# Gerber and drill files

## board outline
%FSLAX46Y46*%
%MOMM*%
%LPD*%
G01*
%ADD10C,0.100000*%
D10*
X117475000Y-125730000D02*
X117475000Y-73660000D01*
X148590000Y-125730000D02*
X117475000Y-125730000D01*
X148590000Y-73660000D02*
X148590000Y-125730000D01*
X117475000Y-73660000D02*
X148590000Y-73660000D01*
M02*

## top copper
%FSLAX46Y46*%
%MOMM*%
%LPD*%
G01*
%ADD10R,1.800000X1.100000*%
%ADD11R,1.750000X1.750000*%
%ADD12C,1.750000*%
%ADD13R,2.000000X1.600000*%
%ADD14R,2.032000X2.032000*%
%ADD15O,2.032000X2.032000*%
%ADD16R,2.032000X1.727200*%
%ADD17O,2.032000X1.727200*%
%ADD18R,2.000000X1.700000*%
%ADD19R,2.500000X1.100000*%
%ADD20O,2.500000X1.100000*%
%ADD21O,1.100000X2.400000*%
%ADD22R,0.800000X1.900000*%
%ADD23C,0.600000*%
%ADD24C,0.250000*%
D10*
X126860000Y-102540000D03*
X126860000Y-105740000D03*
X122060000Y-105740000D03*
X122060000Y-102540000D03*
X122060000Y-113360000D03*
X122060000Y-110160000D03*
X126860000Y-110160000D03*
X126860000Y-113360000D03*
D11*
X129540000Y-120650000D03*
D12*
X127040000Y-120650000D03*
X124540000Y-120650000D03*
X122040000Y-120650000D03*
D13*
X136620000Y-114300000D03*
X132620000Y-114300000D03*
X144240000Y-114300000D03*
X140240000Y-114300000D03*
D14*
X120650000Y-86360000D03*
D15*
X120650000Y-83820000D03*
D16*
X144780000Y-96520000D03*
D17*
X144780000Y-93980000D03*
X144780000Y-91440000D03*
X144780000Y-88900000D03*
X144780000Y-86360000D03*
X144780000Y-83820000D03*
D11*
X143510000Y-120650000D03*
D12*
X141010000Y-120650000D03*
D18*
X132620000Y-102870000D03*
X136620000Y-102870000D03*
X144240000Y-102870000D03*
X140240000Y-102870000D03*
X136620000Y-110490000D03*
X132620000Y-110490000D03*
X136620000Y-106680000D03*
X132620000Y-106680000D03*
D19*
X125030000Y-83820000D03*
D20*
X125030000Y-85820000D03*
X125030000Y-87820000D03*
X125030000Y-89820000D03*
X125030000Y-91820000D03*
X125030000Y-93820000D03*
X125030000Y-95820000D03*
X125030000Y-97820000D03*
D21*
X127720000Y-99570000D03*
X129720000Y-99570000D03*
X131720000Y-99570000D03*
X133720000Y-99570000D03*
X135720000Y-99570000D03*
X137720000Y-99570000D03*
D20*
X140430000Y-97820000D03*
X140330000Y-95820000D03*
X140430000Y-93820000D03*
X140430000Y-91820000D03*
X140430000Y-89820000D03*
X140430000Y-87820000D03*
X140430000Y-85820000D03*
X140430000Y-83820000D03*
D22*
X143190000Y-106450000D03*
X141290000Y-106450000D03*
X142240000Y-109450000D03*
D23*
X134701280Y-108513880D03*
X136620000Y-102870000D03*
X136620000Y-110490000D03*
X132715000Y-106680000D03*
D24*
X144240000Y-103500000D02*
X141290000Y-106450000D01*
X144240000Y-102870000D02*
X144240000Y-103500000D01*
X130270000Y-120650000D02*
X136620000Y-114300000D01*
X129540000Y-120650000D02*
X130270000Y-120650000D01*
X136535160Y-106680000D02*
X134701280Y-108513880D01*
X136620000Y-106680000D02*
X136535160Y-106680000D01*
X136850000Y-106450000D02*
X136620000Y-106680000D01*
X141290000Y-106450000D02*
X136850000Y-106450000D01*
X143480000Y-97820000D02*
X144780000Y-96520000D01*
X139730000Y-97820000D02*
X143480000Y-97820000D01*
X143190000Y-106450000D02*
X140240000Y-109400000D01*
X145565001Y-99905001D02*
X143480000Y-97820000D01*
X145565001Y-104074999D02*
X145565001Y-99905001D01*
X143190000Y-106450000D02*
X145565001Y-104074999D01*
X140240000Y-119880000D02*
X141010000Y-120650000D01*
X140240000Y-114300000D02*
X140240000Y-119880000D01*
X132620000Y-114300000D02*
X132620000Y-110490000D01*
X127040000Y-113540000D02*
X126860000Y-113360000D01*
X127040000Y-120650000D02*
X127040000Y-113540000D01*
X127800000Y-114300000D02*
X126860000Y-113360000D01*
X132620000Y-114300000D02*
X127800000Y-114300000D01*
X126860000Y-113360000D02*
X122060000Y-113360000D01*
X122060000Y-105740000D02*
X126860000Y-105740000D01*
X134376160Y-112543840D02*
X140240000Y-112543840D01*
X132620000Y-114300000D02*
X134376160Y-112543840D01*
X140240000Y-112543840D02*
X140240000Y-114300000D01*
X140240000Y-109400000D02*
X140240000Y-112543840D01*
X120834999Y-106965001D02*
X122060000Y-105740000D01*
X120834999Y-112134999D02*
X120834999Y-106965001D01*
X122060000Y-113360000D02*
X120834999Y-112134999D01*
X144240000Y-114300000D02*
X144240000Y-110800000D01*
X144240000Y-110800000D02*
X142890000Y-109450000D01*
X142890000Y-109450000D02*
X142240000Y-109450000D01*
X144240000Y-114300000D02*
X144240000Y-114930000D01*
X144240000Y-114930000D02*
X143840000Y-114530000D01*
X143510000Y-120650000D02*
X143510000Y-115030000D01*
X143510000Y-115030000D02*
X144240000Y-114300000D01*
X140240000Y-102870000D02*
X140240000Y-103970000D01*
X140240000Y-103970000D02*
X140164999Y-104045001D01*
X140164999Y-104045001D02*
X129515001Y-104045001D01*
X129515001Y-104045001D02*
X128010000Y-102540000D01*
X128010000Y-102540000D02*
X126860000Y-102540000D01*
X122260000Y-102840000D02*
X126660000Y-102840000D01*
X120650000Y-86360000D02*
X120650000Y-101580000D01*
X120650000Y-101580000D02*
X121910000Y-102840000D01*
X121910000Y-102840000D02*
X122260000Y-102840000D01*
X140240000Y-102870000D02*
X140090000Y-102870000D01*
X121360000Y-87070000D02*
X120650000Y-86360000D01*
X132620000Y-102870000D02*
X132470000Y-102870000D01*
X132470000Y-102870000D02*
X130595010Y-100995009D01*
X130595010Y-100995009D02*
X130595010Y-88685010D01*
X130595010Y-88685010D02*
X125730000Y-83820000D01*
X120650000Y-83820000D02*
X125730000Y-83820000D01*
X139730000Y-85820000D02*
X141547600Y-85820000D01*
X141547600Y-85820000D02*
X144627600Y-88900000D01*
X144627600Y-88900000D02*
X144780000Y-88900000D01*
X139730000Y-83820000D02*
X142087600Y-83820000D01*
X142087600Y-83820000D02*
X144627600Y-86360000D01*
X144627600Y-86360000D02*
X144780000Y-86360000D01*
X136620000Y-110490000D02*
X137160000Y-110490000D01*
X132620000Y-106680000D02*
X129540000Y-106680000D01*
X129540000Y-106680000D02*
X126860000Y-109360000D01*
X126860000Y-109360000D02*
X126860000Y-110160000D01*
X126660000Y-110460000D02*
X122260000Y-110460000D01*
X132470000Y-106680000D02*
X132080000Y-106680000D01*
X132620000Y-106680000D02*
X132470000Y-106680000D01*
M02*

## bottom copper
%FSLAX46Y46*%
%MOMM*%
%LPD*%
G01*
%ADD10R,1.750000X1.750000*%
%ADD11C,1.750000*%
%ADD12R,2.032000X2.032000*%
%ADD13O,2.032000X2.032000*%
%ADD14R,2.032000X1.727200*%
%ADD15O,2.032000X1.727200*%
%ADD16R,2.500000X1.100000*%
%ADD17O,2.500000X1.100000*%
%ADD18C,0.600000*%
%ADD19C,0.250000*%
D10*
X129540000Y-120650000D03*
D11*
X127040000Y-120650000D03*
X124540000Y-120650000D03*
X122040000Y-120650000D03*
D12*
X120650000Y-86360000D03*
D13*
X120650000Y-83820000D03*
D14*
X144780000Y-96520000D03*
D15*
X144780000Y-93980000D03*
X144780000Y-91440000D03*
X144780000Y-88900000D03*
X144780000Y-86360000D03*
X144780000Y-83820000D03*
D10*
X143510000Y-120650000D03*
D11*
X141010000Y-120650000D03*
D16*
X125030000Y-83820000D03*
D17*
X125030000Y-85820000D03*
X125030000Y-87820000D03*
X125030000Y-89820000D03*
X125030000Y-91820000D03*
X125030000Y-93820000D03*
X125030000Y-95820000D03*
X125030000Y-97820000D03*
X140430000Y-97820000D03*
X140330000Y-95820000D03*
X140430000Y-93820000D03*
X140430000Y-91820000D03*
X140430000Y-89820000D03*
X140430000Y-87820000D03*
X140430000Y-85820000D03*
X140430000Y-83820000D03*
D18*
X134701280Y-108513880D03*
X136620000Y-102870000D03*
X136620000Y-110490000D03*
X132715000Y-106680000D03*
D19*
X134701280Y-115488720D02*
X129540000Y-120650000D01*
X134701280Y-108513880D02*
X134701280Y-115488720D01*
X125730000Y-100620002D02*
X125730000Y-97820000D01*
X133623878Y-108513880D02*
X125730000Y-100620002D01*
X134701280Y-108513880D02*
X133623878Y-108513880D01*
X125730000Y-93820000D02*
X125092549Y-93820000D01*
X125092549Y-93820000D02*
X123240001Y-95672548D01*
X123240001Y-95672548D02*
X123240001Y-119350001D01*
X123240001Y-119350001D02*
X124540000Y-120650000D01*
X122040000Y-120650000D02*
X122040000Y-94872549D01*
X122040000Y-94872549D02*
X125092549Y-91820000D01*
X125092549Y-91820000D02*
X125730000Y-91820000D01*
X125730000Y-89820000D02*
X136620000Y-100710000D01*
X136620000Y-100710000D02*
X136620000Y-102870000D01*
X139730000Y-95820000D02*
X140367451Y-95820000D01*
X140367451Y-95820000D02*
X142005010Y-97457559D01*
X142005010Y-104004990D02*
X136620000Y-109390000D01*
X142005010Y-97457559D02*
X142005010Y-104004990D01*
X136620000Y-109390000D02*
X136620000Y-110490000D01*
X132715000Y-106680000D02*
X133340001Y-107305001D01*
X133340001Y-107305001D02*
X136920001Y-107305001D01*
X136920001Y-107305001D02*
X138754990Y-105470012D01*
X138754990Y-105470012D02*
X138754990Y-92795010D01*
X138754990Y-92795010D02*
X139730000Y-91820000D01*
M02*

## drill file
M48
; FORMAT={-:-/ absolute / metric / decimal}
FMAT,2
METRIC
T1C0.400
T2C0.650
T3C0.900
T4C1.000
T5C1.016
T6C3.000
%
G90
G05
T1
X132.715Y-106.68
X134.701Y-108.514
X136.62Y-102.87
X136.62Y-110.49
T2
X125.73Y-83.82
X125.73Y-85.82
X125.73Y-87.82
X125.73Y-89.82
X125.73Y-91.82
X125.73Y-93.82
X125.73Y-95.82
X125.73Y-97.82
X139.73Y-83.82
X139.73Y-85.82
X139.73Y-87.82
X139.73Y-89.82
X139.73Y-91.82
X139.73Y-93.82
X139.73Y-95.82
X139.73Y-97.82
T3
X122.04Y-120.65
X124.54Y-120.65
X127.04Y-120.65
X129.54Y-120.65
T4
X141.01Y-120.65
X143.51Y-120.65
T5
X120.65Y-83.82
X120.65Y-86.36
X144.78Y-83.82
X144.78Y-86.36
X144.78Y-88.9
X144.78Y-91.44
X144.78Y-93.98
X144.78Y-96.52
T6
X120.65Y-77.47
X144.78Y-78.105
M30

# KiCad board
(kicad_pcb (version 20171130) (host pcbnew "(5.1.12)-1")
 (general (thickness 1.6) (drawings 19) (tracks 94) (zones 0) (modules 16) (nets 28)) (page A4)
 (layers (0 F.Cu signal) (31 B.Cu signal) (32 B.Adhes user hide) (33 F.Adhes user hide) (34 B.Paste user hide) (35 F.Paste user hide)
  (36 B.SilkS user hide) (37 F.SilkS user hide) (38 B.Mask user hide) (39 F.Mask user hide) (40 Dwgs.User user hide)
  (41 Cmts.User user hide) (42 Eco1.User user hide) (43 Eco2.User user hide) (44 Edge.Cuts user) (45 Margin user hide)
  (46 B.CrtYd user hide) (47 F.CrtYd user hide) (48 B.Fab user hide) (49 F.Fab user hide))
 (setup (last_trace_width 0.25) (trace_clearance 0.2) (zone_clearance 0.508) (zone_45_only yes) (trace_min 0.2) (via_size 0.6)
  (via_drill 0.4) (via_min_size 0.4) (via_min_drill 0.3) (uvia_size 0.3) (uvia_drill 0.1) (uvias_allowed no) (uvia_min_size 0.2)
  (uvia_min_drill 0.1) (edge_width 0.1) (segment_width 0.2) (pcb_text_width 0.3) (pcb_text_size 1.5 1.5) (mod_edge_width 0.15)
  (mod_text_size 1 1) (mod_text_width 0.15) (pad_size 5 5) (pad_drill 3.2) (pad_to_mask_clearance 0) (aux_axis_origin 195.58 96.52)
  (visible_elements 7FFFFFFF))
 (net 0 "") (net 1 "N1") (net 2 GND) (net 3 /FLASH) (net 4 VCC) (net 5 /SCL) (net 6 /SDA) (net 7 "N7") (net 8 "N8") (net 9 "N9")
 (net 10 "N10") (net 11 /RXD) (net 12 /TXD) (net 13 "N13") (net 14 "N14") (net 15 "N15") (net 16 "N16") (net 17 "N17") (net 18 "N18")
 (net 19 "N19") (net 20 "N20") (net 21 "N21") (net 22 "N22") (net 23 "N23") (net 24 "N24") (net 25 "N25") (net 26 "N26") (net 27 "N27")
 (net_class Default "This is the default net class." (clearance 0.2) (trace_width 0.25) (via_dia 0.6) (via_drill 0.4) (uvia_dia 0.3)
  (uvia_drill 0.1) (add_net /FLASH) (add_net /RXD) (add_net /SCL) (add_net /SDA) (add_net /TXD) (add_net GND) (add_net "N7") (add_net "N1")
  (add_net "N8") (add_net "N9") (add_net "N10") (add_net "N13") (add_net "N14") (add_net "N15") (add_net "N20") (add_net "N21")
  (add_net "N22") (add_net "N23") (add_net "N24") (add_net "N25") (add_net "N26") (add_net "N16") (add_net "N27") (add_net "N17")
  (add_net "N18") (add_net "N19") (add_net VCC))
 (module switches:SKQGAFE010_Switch (layer F.Cu) (at 124.46 104.14 180)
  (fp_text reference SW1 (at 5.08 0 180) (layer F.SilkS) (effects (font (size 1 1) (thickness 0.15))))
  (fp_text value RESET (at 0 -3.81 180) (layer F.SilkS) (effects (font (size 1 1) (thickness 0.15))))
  (pad 3 smd rect (at -2.4 1.6 180) (size 1.8 1.1) (layers F.Cu F.Paste F.Mask) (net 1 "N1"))
  (pad 1 smd rect (at -2.4 -1.6 180) (size 1.8 1.1) (layers F.Cu F.Paste F.Mask) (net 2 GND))
  (pad 2 smd rect (at 2.4 -1.6 180) (size 1.8 1.1) (layers F.Cu F.Paste F.Mask) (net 2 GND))
  (pad 4 smd rect (at 2.4 1.6 180) (size 1.8 1.1) (layers F.Cu F.Paste F.Mask) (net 1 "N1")))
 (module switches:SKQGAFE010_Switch (layer F.Cu) (at 124.46 111.76)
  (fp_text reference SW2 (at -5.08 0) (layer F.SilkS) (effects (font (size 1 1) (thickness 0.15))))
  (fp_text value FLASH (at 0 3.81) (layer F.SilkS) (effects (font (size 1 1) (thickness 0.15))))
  (pad 3 smd rect (at -2.4 1.6) (size 1.8 1.1) (layers F.Cu F.Paste F.Mask) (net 2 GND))
  (pad 1 smd rect (at -2.4 -1.6) (size 1.8 1.1) (layers F.Cu F.Paste F.Mask) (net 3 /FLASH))
  (pad 2 smd rect (at 2.4 -1.6) (size 1.8 1.1) (layers F.Cu F.Paste F.Mask) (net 3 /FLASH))
  (pad 4 smd rect (at 2.4 1.6) (size 1.8 1.1) (layers F.Cu F.Paste F.Mask) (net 2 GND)))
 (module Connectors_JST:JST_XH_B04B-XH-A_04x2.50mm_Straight (layer F.Cu) (at 129.54 120.65 180)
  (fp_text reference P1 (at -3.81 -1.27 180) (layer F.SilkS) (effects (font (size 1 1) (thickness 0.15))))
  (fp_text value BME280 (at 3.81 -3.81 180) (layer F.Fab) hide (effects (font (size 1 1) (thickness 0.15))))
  (pad 1 thru_hole rect (at 0 0 180) (size 1.75 1.75) (drill 0.9) (layers *.Cu *.Mask) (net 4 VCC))
  (pad 2 thru_hole circle (at 2.5 0 180) (size 1.75 1.75) (drill 0.9) (layers *.Cu *.Mask) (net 2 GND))
  (pad 3 thru_hole circle (at 5 0 180) (size 1.75 1.75) (drill 0.9) (layers *.Cu *.Mask) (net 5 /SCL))
  (pad 4 thru_hole circle (at 7.5 0 180) (size 1.75 1.75) (drill 0.9) (layers *.Cu *.Mask) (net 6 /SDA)))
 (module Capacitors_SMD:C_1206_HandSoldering (layer F.Cu) (at 134.62 114.3 180)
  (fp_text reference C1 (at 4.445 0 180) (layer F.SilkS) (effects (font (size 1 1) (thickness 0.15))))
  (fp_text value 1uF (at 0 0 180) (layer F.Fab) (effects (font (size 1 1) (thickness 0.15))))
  (pad 1 smd rect (at -2 0 180) (size 2 1.6) (layers F.Cu F.Paste F.Mask) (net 4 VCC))
  (pad 2 smd rect (at 2 0 180) (size 2 1.6) (layers F.Cu F.Paste F.Mask) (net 2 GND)))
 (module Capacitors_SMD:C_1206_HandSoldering (layer F.Cu) (at 142.24 114.3 180)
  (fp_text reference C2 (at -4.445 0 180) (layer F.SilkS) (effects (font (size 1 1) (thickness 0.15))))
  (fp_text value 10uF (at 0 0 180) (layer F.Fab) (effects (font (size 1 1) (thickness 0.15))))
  (pad 1 smd rect (at -2 0 180) (size 2 1.6) (layers F.Cu F.Paste F.Mask) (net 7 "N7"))
  (pad 2 smd rect (at 2 0 180) (size 2 1.6) (layers F.Cu F.Paste F.Mask) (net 2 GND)))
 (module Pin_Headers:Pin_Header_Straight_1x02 (layer F.Cu) (at 120.65 86.36 180)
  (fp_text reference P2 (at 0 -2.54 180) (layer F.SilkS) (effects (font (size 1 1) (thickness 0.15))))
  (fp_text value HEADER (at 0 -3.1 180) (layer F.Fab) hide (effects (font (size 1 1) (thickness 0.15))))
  (pad 1 thru_hole rect (at 0 0 180) (size 2.032 2.032) (drill 1.016) (layers *.Cu *.Mask) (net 1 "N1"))
  (pad 2 thru_hole oval (at 0 2.54 180) (size 2.032 2.032) (drill 1.016) (layers *.Cu *.Mask) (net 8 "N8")))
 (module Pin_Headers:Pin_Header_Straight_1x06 (layer F.Cu) (at 144.78 96.52 180)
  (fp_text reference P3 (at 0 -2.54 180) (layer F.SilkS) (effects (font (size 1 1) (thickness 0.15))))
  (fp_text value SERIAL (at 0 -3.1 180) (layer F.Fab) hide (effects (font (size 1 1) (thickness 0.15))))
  (pad 1 thru_hole rect (at 0 0 180) (size 2.032 1.7272) (drill 1.016) (layers *.Cu *.Mask) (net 2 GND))
  (pad 2 thru_hole oval (at 0 2.54 180) (size 2.032 1.7272) (drill 1.016) (layers *.Cu *.Mask) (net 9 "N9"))
  (pad 3 thru_hole oval (at 0 5.08 180) (size 2.032 1.7272) (drill 1.016) (layers *.Cu *.Mask) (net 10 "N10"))
  (pad 4 thru_hole oval (at 0 7.62 180) (size 2.032 1.7272) (drill 1.016) (layers *.Cu *.Mask) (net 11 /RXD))
  (pad 5 thru_hole oval (at 0 10.16 180) (size 2.032 1.7272) (drill 1.016) (layers *.Cu *.Mask) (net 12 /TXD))
  (pad 6 thru_hole oval (at 0 12.7 180) (size 2.032 1.7272) (drill 1.016) (layers *.Cu *.Mask) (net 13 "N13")))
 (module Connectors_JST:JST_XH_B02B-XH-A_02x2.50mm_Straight (layer F.Cu) (at 143.51 120.65 180)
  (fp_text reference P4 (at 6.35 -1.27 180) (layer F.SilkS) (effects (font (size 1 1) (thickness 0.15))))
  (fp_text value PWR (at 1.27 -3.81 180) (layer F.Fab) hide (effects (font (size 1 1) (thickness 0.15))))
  (pad 1 thru_hole rect (at 0 0 180) (size 1.75 1.75) (drill 1) (layers *.Cu *.Mask) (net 7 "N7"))
  (pad 2 thru_hole circle (at 2.5 0 180) (size 1.75 1.75) (drill 1) (layers *.Cu *.Mask) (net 2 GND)))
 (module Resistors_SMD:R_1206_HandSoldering (layer F.Cu) (at 134.62 102.87)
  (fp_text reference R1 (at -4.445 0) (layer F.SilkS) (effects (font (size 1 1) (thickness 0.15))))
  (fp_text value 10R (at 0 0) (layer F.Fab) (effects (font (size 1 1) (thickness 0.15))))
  (pad 1 smd rect (at -2 0) (size 2 1.7) (layers F.Cu F.Paste F.Mask) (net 8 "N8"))
  (pad 2 smd rect (at 2 0) (size 2 1.7) (layers F.Cu F.Paste F.Mask) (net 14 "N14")))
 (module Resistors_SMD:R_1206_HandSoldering (layer F.Cu) (at 142.24 102.87 180)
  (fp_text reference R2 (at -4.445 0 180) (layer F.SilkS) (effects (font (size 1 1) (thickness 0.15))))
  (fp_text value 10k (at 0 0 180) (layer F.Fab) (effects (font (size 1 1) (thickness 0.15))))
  (pad 1 smd rect (at -2 0 180) (size 2 1.7) (layers F.Cu F.Paste F.Mask) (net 4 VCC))
  (pad 2 smd rect (at 2 0 180) (size 2 1.7) (layers F.Cu F.Paste F.Mask) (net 1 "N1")))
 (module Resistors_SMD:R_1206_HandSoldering (layer F.Cu) (at 134.62 110.49 180)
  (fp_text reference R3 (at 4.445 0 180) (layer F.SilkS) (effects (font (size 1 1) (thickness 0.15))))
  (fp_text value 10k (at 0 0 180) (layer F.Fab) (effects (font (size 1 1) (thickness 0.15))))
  (pad 1 smd rect (at -2 0 180) (size 2 1.7) (layers F.Cu F.Paste F.Mask) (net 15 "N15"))
  (pad 2 smd rect (at 2 0 180) (size 2 1.7) (layers F.Cu F.Paste F.Mask) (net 2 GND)))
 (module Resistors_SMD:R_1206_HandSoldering (layer F.Cu) (at 134.62 106.68 180)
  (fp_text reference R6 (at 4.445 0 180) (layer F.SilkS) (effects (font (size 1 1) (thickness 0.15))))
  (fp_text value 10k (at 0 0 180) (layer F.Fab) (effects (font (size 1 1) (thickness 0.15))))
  (pad 1 smd rect (at -2 0 180) (size 2 1.7) (layers F.Cu F.Paste F.Mask) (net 4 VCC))
  (pad 2 smd rect (at 2 0 180) (size 2 1.7) (layers F.Cu F.Paste F.Mask) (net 3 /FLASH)))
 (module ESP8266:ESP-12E (layer F.Cu) (at 125.73 83.82)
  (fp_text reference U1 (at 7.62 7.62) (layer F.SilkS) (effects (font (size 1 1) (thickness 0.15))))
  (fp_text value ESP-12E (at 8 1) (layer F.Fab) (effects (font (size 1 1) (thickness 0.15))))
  (pad 1 thru_hole rect (at 0 0) (size 2.5 1.1) (drill 0.65 (offset -0.7 0)) (layers *.Cu *.Mask F.SilkS) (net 8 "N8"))
  (pad 2 thru_hole oval (at 0 2) (size 2.5 1.1) (drill 0.65 (offset -0.7 0)) (layers *.Cu *.Mask F.SilkS) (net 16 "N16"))
  (pad 3 thru_hole oval (at 0 4) (size 2.5 1.1) (drill 0.65 (offset -0.7 0)) (layers *.Cu *.Mask F.SilkS) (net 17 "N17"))
  (pad 4 thru_hole oval (at 0 6) (size 2.5 1.1) (drill 0.65 (offset -0.7 0)) (layers *.Cu *.Mask F.SilkS) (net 14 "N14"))
  (pad 5 thru_hole oval (at 0 8) (size 2.5 1.1) (drill 0.65 (offset -0.7 0)) (layers *.Cu *.Mask F.SilkS) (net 6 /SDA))
  (pad 6 thru_hole oval (at 0 10) (size 2.5 1.1) (drill 0.65 (offset -0.7 0)) (layers *.Cu *.Mask F.SilkS) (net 5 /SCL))
  (pad 7 thru_hole oval (at 0 12) (size 2.5 1.1) (drill 0.65 (offset -0.7 0)) (layers *.Cu *.Mask F.SilkS) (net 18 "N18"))
  (pad 8 thru_hole oval (at 0 14) (size 2.5 1.1) (drill 0.65 (offset -0.7 0)) (layers *.Cu *.Mask F.SilkS) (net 4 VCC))
  (pad 9 smd oval (at 1.99 15.75 90) (size 2.4 1.1) (layers F.Cu F.Paste F.Mask) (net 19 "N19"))
  (pad 10 smd oval (at 3.99 15.75 90) (size 2.4 1.1) (layers F.Cu F.Paste F.Mask) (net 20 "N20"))
  (pad 11 smd oval (at 5.99 15.75 90) (size 2.4 1.1) (layers F.Cu F.Paste F.Mask) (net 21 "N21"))
  (pad 12 smd oval (at 7.99 15.75 90) (size 2.4 1.1) (layers F.Cu F.Paste F.Mask) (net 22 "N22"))
  (pad 13 smd oval (at 9.99 15.75 90) (size 2.4 1.1) (layers F.Cu F.Paste F.Mask) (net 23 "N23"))
  (pad 14 smd oval (at 11.99 15.75 90) (size 2.4 1.1) (layers F.Cu F.Paste F.Mask) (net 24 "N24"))
  (pad 15 thru_hole oval (at 14 14) (size 2.5 1.1) (drill 0.65 (offset 0.7 0)) (layers *.Cu *.Mask F.SilkS) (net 2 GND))
  (pad 16 thru_hole oval (at 14 12) (size 2.5 1.1) (drill 0.65 (offset 0.6 0)) (layers *.Cu *.Mask F.SilkS) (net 15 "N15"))
  (pad 17 thru_hole oval (at 14 10) (size 2.5 1.1) (drill 0.65 (offset 0.7 0)) (layers *.Cu *.Mask F.SilkS) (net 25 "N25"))
  (pad 18 thru_hole oval (at 14 8) (size 2.5 1.1) (drill 0.65 (offset 0.7 0)) (layers *.Cu *.Mask F.SilkS) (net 3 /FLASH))
  (pad 19 thru_hole oval (at 14 6) (size 2.5 1.1) (drill 0.65 (offset 0.7 0)) (layers *.Cu *.Mask F.SilkS) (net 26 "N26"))
  (pad 20 thru_hole oval (at 14 4) (size 2.5 1.1) (drill 0.65 (offset 0.7 0)) (layers *.Cu *.Mask F.SilkS) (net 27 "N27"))
  (pad 21 thru_hole oval (at 14 2) (size 2.5 1.1) (drill 0.65 (offset 0.7 0)) (layers *.Cu *.Mask F.SilkS) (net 11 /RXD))
  (pad 22 thru_hole oval (at 14 0) (size 2.5 1.1) (drill 0.65 (offset 0.7 0)) (layers *.Cu *.Mask F.SilkS) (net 12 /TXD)))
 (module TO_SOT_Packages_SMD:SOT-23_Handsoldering (layer F.Cu) (at 142.24 107.95 270)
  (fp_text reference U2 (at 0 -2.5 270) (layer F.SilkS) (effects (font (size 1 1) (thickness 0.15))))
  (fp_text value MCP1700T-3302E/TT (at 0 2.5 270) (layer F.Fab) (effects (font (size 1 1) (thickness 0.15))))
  (pad 1 smd rect (at -1.5 -0.95 270) (size 1.9 0.8) (layers F.Cu F.Paste F.Mask) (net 2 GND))
  (pad 2 smd rect (at -1.5 0.95 270) (size 1.9 0.8) (layers F.Cu F.Paste F.Mask) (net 4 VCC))
  (pad 3 smd rect (at 1.5 0 270) (size 1.9 0.8) (layers F.Cu F.Paste F.Mask) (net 7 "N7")))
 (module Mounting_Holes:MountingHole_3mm (layer F.Cu) (at 144.78 78.105)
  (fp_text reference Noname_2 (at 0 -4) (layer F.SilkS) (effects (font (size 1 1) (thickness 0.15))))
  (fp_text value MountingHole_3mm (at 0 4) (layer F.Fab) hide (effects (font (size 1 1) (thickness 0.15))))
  (pad 1 np_thru_hole circle (at 0 0) (size 3 3) (drill 3) (layers *.Cu *.Mask)))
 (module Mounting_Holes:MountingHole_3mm (layer F.Cu) (at 120.65 77.47)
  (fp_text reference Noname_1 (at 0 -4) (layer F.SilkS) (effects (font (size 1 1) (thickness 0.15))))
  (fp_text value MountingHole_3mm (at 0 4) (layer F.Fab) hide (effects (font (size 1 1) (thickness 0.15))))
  (pad 1 np_thru_hole circle (at 0 0) (size 3 3) (drill 3) (layers *.Cu *.Mask)))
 (gr_line (start 117.475 125.73) (end 117.475 73.66) (angle 90) (layer Edge.Cuts) (width 0.1))
 (gr_line (start 148.59 125.73) (end 117.475 125.73) (angle 90) (layer Edge.Cuts) (width 0.1))
 (gr_line (start 148.59 73.66) (end 148.59 125.73) (angle 90) (layer Edge.Cuts) (width 0.1))
 (gr_line (start 117.475 73.66) (end 148.59 73.66) (angle 90) (layer Edge.Cuts) (width 0.1))
 (via (at 134.70128 108.51388) (size 0.6) (drill 0.4) (layers F.Cu B.Cu) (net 4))
 (segment (start 144.24 103.5) (end 141.29 106.45) (width 0.25) (layer F.Cu) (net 4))
 (segment (start 144.24 102.87) (end 144.24 103.5) (width 0.25) (layer F.Cu) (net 4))
 (segment (start 130.27 120.65) (end 136.62 114.3) (width 0.25) (layer F.Cu) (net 4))
 (segment (start 129.54 120.65) (end 130.27 120.65) (width 0.25) (layer F.Cu) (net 4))
 (segment (start 136.53516 106.68) (end 134.70128 108.51388) (width 0.25) (layer F.Cu) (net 4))
 (segment (start 136.62 106.68) (end 136.53516 106.68) (width 0.25) (layer F.Cu) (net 4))
 (segment (start 134.70128 115.48872) (end 129.54 120.65) (width 0.25) (layer B.Cu) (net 4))
 (segment (start 134.70128 108.51388) (end 134.70128 115.48872) (width 0.25) (layer B.Cu) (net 4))
 (segment (start 125.73 100.620002) (end 125.73 97.82) (width 0.25) (layer B.Cu) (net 4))
 (segment (start 133.623878 108.51388) (end 125.73 100.620002) (width 0.25) (layer B.Cu) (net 4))
 (segment (start 134.70128 108.51388) (end 133.623878 108.51388) (width 0.25) (layer B.Cu) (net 4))
 (segment (start 136.85 106.45) (end 136.62 106.68) (width 0.25) (layer F.Cu) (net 4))
 (segment (start 141.29 106.45) (end 136.85 106.45) (width 0.25) (layer F.Cu) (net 4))
 (segment (start 143.48 97.82) (end 144.78 96.52) (width 0.25) (layer F.Cu) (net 2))
 (segment (start 139.73 97.82) (end 143.48 97.82) (width 0.25) (layer F.Cu) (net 2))
 (segment (start 143.19 106.45) (end 140.24 109.4) (width 0.25) (layer F.Cu) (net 2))
 (segment (start 145.565001 99.905001) (end 143.48 97.82) (width 0.25) (layer F.Cu) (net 2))
 (segment (start 145.565001 104.074999) (end 145.565001 99.905001) (width 0.25) (layer F.Cu) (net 2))
 (segment (start 143.19 106.45) (end 145.565001 104.074999) (width 0.25) (layer F.Cu) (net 2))
 (segment (start 140.24 119.88) (end 141.01 120.65) (width 0.25) (layer F.Cu) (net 2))
 (segment (start 140.24 114.3) (end 140.24 119.88) (width 0.25) (layer F.Cu) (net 2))
 (segment (start 132.62 114.3) (end 132.62 110.49) (width 0.25) (layer F.Cu) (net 2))
 (segment (start 127.04 113.54) (end 126.86 113.36) (width 0.25) (layer F.Cu) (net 2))
 (segment (start 127.04 120.65) (end 127.04 113.54) (width 0.25) (layer F.Cu) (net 2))
 (segment (start 127.8 114.3) (end 126.86 113.36) (width 0.25) (layer F.Cu) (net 2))
 (segment (start 132.62 114.3) (end 127.8 114.3) (width 0.25) (layer F.Cu) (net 2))
 (segment (start 126.86 113.36) (end 122.06 113.36) (width 0.25) (layer F.Cu) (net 2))
 (segment (start 122.06 105.74) (end 126.86 105.74) (width 0.25) (layer F.Cu) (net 2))
 (segment (start 134.37616 112.54384) (end 140.24 112.54384) (width 0.25) (layer F.Cu) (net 2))
 (segment (start 132.62 114.3) (end 134.37616 112.54384) (width 0.25) (layer F.Cu) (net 2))
 (segment (start 140.24 112.54384) (end 140.24 114.3) (width 0.25) (layer F.Cu) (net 2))
 (segment (start 140.24 109.4) (end 140.24 112.54384) (width 0.25) (layer F.Cu) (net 2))
 (segment (start 120.834999 106.965001) (end 122.06 105.74) (width 0.25) (layer F.Cu) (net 2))
 (segment (start 120.834999 112.134999) (end 120.834999 106.965001) (width 0.25) (layer F.Cu) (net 2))
 (segment (start 122.06 113.36) (end 120.834999 112.134999) (width 0.25) (layer F.Cu) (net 2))
 (segment (start 144.24 114.3) (end 144.24 110.8) (width 0.25) (layer F.Cu) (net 7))
 (segment (start 144.24 110.8) (end 142.89 109.45) (width 0.25) (layer F.Cu) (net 7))
 (segment (start 142.89 109.45) (end 142.24 109.45) (width 0.25) (layer F.Cu) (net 7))
 (segment (start 144.24 114.3) (end 144.24 114.93) (width 0.25) (layer F.Cu) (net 7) (status 30))
 (segment (start 144.24 114.93) (end 143.84 114.53) (width 0.25) (layer F.Cu) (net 7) (status 30))
 (segment (start 143.51 120.65) (end 143.51 115.03) (width 0.25) (layer F.Cu) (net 7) (status 30))
 (segment (start 143.51 115.03) (end 144.24 114.3) (width 0.25) (layer F.Cu) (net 7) (status 30))
 (segment (start 125.73 93.82) (end 125.092549 93.82) (width 0.25) (layer B.Cu) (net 5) (status 30))
 (segment (start 125.092549 93.82) (end 123.240001 95.672548) (width 0.25) (layer B.Cu) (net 5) (status 10))
 (segment (start 123.240001 95.672548) (end 123.240001 119.350001) (width 0.25) (layer B.Cu) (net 5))
 (segment (start 123.240001 119.350001) (end 124.54 120.65) (width 0.25) (layer B.Cu) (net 5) (status 20))
 (segment (start 122.04 120.65) (end 122.04 94.872549) (width 0.25) (layer B.Cu) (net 6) (status 10))
 (segment (start 122.04 94.872549) (end 125.092549 91.82) (width 0.25) (layer B.Cu) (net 6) (status 20))
 (segment (start 125.092549 91.82) (end 125.73 91.82) (width 0.25) (layer B.Cu) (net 6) (status 30))
 (segment (start 140.24 102.87) (end 140.24 103.97) (width 0.25) (layer F.Cu) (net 1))
 (segment (start 140.24 103.97) (end 140.164999 104.045001) (width 0.25) (layer F.Cu) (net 1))
 (segment (start 140.164999 104.045001) (end 129.515001 104.045001) (width 0.25) (layer F.Cu) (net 1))
 (segment (start 129.515001 104.045001) (end 128.01 102.54) (width 0.25) (layer F.Cu) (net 1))
 (segment (start 128.01 102.54) (end 126.86 102.54) (width 0.25) (layer F.Cu) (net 1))
 (segment (start 122.26 102.84) (end 126.66 102.84) (width 0.25) (layer F.Cu) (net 1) (status 30))
 (segment (start 120.65 86.36) (end 120.65 101.58) (width 0.25) (layer F.Cu) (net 1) (status 10))
 (segment (start 120.65 101.58) (end 121.91 102.84) (width 0.25) (layer F.Cu) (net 1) (status 20))
 (segment (start 121.91 102.84) (end 122.26 102.84) (width 0.25) (layer F.Cu) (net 1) (status 30))
 (segment (start 140.24 102.87) (end 140.09 102.87) (width 0.25) (layer F.Cu) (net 1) (status 30))
 (segment (start 121.36 87.07) (end 120.65 86.36) (width 0.25) (layer F.Cu) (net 1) (status 30))
 (segment (start 132.62 102.87) (end 132.47 102.87) (width 0.25) (layer F.Cu) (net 8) (status 30))
 (segment (start 132.47 102.87) (end 130.59501 100.995009) (width 0.25) (layer F.Cu) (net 8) (status 10))
 (segment (start 130.59501 100.995009) (end 130.59501 88.68501) (width 0.25) (layer F.Cu) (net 8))
 (segment (start 130.59501 88.68501) (end 125.73 83.82) (width 0.25) (layer F.Cu) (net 8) (status 20))
 (segment (start 120.65 83.82) (end 125.73 83.82) (width 0.25) (layer F.Cu) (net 8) (status 30))
 (segment (start 139.73 85.82) (end 141.5476 85.82) (width 0.25) (layer F.Cu) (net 11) (status 30))
 (segment (start 141.5476 85.82) (end 144.6276 88.9) (width 0.25) (layer F.Cu) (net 11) (status 20))
 (segment (start 144.6276 88.9) (end 144.78 88.9) (width 0.25) (layer F.Cu) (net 11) (status 30))
 (segment (start 139.73 83.82) (end 142.0876 83.82) (width 0.25) (layer F.Cu) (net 12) (status 10))
 (segment (start 142.0876 83.82) (end 144.6276 86.36) (width 0.25) (layer F.Cu) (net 12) (status 20))
 (segment (start 144.6276 86.36) (end 144.78 86.36) (width 0.25) (layer F.Cu) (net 12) (status 30))
 (via (at 136.62 102.87) (size 0.6) (drill 0.4) (layers F.Cu B.Cu) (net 14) (status 30))
 (segment (start 125.73 89.82) (end 136.62 100.71) (width 0.25) (layer B.Cu) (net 14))
 (segment (start 136.62 100.71) (end 136.62 102.87) (width 0.25) (layer B.Cu) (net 14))
 (via (at 136.62 110.49) (size 0.6) (drill 0.4) (layers F.Cu B.Cu) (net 15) (status 30))
 (segment (start 139.73 95.82) (end 140.367451 95.82) (width 0.25) (layer B.Cu) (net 15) (status 30))
 (segment (start 140.367451 95.82) (end 142.00501 97.457559) (width 0.25) (layer B.Cu) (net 15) (status 10))
 (segment (start 142.00501 104.00499) (end 136.62 109.39) (width 0.25) (layer B.Cu) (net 15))
 (segment (start 142.00501 97.457559) (end 142.00501 104.00499) (width 0.25) (layer B.Cu) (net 15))
 (segment (start 136.62 109.39) (end 136.62 110.49) (width 0.25) (layer B.Cu) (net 15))
 (segment (start 136.62 110.49) (end 137.16 110.49) (width 0.25) (layer F.Cu) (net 15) (status 30))
 (via (at 132.715 106.68) (size 0.6) (drill 0.4) (layers F.Cu B.Cu) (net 3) (status 30))
 (segment (start 132.715 106.68) (end 133.340001 107.305001) (width 0.25) (layer B.Cu) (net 3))
 (segment (start 133.340001 107.305001) (end 136.920001 107.305001) (width 0.25) (layer B.Cu) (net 3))
 (segment (start 136.920001 107.305001) (end 138.75499 105.470012) (width 0.25) (layer B.Cu) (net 3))
 (segment (start 138.75499 105.470012) (end 138.75499 92.79501) (width 0.25) (layer B.Cu) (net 3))
 (segment (start 138.75499 92.79501) (end 139.73 91.82) (width 0.25) (layer B.Cu) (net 3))
 (segment (start 132.62 106.68) (end 129.54 106.68) (width 0.25) (layer F.Cu) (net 3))
 (segment (start 129.54 106.68) (end 126.86 109.36) (width 0.25) (layer F.Cu) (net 3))
 (segment (start 126.86 109.36) (end 126.86 110.16) (width 0.25) (layer F.Cu) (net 3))
 (segment (start 126.66 110.46) (end 122.26 110.46) (width 0.25) (layer F.Cu) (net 3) (status 30))
 (segment (start 132.47 106.68) (end 132.08 106.68) (width 0.25) (layer F.Cu) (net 3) (status 30))
 (segment (start 132.62 106.68) (end 132.47 106.68) (width 0.25) (layer F.Cu) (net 3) (status 30)))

